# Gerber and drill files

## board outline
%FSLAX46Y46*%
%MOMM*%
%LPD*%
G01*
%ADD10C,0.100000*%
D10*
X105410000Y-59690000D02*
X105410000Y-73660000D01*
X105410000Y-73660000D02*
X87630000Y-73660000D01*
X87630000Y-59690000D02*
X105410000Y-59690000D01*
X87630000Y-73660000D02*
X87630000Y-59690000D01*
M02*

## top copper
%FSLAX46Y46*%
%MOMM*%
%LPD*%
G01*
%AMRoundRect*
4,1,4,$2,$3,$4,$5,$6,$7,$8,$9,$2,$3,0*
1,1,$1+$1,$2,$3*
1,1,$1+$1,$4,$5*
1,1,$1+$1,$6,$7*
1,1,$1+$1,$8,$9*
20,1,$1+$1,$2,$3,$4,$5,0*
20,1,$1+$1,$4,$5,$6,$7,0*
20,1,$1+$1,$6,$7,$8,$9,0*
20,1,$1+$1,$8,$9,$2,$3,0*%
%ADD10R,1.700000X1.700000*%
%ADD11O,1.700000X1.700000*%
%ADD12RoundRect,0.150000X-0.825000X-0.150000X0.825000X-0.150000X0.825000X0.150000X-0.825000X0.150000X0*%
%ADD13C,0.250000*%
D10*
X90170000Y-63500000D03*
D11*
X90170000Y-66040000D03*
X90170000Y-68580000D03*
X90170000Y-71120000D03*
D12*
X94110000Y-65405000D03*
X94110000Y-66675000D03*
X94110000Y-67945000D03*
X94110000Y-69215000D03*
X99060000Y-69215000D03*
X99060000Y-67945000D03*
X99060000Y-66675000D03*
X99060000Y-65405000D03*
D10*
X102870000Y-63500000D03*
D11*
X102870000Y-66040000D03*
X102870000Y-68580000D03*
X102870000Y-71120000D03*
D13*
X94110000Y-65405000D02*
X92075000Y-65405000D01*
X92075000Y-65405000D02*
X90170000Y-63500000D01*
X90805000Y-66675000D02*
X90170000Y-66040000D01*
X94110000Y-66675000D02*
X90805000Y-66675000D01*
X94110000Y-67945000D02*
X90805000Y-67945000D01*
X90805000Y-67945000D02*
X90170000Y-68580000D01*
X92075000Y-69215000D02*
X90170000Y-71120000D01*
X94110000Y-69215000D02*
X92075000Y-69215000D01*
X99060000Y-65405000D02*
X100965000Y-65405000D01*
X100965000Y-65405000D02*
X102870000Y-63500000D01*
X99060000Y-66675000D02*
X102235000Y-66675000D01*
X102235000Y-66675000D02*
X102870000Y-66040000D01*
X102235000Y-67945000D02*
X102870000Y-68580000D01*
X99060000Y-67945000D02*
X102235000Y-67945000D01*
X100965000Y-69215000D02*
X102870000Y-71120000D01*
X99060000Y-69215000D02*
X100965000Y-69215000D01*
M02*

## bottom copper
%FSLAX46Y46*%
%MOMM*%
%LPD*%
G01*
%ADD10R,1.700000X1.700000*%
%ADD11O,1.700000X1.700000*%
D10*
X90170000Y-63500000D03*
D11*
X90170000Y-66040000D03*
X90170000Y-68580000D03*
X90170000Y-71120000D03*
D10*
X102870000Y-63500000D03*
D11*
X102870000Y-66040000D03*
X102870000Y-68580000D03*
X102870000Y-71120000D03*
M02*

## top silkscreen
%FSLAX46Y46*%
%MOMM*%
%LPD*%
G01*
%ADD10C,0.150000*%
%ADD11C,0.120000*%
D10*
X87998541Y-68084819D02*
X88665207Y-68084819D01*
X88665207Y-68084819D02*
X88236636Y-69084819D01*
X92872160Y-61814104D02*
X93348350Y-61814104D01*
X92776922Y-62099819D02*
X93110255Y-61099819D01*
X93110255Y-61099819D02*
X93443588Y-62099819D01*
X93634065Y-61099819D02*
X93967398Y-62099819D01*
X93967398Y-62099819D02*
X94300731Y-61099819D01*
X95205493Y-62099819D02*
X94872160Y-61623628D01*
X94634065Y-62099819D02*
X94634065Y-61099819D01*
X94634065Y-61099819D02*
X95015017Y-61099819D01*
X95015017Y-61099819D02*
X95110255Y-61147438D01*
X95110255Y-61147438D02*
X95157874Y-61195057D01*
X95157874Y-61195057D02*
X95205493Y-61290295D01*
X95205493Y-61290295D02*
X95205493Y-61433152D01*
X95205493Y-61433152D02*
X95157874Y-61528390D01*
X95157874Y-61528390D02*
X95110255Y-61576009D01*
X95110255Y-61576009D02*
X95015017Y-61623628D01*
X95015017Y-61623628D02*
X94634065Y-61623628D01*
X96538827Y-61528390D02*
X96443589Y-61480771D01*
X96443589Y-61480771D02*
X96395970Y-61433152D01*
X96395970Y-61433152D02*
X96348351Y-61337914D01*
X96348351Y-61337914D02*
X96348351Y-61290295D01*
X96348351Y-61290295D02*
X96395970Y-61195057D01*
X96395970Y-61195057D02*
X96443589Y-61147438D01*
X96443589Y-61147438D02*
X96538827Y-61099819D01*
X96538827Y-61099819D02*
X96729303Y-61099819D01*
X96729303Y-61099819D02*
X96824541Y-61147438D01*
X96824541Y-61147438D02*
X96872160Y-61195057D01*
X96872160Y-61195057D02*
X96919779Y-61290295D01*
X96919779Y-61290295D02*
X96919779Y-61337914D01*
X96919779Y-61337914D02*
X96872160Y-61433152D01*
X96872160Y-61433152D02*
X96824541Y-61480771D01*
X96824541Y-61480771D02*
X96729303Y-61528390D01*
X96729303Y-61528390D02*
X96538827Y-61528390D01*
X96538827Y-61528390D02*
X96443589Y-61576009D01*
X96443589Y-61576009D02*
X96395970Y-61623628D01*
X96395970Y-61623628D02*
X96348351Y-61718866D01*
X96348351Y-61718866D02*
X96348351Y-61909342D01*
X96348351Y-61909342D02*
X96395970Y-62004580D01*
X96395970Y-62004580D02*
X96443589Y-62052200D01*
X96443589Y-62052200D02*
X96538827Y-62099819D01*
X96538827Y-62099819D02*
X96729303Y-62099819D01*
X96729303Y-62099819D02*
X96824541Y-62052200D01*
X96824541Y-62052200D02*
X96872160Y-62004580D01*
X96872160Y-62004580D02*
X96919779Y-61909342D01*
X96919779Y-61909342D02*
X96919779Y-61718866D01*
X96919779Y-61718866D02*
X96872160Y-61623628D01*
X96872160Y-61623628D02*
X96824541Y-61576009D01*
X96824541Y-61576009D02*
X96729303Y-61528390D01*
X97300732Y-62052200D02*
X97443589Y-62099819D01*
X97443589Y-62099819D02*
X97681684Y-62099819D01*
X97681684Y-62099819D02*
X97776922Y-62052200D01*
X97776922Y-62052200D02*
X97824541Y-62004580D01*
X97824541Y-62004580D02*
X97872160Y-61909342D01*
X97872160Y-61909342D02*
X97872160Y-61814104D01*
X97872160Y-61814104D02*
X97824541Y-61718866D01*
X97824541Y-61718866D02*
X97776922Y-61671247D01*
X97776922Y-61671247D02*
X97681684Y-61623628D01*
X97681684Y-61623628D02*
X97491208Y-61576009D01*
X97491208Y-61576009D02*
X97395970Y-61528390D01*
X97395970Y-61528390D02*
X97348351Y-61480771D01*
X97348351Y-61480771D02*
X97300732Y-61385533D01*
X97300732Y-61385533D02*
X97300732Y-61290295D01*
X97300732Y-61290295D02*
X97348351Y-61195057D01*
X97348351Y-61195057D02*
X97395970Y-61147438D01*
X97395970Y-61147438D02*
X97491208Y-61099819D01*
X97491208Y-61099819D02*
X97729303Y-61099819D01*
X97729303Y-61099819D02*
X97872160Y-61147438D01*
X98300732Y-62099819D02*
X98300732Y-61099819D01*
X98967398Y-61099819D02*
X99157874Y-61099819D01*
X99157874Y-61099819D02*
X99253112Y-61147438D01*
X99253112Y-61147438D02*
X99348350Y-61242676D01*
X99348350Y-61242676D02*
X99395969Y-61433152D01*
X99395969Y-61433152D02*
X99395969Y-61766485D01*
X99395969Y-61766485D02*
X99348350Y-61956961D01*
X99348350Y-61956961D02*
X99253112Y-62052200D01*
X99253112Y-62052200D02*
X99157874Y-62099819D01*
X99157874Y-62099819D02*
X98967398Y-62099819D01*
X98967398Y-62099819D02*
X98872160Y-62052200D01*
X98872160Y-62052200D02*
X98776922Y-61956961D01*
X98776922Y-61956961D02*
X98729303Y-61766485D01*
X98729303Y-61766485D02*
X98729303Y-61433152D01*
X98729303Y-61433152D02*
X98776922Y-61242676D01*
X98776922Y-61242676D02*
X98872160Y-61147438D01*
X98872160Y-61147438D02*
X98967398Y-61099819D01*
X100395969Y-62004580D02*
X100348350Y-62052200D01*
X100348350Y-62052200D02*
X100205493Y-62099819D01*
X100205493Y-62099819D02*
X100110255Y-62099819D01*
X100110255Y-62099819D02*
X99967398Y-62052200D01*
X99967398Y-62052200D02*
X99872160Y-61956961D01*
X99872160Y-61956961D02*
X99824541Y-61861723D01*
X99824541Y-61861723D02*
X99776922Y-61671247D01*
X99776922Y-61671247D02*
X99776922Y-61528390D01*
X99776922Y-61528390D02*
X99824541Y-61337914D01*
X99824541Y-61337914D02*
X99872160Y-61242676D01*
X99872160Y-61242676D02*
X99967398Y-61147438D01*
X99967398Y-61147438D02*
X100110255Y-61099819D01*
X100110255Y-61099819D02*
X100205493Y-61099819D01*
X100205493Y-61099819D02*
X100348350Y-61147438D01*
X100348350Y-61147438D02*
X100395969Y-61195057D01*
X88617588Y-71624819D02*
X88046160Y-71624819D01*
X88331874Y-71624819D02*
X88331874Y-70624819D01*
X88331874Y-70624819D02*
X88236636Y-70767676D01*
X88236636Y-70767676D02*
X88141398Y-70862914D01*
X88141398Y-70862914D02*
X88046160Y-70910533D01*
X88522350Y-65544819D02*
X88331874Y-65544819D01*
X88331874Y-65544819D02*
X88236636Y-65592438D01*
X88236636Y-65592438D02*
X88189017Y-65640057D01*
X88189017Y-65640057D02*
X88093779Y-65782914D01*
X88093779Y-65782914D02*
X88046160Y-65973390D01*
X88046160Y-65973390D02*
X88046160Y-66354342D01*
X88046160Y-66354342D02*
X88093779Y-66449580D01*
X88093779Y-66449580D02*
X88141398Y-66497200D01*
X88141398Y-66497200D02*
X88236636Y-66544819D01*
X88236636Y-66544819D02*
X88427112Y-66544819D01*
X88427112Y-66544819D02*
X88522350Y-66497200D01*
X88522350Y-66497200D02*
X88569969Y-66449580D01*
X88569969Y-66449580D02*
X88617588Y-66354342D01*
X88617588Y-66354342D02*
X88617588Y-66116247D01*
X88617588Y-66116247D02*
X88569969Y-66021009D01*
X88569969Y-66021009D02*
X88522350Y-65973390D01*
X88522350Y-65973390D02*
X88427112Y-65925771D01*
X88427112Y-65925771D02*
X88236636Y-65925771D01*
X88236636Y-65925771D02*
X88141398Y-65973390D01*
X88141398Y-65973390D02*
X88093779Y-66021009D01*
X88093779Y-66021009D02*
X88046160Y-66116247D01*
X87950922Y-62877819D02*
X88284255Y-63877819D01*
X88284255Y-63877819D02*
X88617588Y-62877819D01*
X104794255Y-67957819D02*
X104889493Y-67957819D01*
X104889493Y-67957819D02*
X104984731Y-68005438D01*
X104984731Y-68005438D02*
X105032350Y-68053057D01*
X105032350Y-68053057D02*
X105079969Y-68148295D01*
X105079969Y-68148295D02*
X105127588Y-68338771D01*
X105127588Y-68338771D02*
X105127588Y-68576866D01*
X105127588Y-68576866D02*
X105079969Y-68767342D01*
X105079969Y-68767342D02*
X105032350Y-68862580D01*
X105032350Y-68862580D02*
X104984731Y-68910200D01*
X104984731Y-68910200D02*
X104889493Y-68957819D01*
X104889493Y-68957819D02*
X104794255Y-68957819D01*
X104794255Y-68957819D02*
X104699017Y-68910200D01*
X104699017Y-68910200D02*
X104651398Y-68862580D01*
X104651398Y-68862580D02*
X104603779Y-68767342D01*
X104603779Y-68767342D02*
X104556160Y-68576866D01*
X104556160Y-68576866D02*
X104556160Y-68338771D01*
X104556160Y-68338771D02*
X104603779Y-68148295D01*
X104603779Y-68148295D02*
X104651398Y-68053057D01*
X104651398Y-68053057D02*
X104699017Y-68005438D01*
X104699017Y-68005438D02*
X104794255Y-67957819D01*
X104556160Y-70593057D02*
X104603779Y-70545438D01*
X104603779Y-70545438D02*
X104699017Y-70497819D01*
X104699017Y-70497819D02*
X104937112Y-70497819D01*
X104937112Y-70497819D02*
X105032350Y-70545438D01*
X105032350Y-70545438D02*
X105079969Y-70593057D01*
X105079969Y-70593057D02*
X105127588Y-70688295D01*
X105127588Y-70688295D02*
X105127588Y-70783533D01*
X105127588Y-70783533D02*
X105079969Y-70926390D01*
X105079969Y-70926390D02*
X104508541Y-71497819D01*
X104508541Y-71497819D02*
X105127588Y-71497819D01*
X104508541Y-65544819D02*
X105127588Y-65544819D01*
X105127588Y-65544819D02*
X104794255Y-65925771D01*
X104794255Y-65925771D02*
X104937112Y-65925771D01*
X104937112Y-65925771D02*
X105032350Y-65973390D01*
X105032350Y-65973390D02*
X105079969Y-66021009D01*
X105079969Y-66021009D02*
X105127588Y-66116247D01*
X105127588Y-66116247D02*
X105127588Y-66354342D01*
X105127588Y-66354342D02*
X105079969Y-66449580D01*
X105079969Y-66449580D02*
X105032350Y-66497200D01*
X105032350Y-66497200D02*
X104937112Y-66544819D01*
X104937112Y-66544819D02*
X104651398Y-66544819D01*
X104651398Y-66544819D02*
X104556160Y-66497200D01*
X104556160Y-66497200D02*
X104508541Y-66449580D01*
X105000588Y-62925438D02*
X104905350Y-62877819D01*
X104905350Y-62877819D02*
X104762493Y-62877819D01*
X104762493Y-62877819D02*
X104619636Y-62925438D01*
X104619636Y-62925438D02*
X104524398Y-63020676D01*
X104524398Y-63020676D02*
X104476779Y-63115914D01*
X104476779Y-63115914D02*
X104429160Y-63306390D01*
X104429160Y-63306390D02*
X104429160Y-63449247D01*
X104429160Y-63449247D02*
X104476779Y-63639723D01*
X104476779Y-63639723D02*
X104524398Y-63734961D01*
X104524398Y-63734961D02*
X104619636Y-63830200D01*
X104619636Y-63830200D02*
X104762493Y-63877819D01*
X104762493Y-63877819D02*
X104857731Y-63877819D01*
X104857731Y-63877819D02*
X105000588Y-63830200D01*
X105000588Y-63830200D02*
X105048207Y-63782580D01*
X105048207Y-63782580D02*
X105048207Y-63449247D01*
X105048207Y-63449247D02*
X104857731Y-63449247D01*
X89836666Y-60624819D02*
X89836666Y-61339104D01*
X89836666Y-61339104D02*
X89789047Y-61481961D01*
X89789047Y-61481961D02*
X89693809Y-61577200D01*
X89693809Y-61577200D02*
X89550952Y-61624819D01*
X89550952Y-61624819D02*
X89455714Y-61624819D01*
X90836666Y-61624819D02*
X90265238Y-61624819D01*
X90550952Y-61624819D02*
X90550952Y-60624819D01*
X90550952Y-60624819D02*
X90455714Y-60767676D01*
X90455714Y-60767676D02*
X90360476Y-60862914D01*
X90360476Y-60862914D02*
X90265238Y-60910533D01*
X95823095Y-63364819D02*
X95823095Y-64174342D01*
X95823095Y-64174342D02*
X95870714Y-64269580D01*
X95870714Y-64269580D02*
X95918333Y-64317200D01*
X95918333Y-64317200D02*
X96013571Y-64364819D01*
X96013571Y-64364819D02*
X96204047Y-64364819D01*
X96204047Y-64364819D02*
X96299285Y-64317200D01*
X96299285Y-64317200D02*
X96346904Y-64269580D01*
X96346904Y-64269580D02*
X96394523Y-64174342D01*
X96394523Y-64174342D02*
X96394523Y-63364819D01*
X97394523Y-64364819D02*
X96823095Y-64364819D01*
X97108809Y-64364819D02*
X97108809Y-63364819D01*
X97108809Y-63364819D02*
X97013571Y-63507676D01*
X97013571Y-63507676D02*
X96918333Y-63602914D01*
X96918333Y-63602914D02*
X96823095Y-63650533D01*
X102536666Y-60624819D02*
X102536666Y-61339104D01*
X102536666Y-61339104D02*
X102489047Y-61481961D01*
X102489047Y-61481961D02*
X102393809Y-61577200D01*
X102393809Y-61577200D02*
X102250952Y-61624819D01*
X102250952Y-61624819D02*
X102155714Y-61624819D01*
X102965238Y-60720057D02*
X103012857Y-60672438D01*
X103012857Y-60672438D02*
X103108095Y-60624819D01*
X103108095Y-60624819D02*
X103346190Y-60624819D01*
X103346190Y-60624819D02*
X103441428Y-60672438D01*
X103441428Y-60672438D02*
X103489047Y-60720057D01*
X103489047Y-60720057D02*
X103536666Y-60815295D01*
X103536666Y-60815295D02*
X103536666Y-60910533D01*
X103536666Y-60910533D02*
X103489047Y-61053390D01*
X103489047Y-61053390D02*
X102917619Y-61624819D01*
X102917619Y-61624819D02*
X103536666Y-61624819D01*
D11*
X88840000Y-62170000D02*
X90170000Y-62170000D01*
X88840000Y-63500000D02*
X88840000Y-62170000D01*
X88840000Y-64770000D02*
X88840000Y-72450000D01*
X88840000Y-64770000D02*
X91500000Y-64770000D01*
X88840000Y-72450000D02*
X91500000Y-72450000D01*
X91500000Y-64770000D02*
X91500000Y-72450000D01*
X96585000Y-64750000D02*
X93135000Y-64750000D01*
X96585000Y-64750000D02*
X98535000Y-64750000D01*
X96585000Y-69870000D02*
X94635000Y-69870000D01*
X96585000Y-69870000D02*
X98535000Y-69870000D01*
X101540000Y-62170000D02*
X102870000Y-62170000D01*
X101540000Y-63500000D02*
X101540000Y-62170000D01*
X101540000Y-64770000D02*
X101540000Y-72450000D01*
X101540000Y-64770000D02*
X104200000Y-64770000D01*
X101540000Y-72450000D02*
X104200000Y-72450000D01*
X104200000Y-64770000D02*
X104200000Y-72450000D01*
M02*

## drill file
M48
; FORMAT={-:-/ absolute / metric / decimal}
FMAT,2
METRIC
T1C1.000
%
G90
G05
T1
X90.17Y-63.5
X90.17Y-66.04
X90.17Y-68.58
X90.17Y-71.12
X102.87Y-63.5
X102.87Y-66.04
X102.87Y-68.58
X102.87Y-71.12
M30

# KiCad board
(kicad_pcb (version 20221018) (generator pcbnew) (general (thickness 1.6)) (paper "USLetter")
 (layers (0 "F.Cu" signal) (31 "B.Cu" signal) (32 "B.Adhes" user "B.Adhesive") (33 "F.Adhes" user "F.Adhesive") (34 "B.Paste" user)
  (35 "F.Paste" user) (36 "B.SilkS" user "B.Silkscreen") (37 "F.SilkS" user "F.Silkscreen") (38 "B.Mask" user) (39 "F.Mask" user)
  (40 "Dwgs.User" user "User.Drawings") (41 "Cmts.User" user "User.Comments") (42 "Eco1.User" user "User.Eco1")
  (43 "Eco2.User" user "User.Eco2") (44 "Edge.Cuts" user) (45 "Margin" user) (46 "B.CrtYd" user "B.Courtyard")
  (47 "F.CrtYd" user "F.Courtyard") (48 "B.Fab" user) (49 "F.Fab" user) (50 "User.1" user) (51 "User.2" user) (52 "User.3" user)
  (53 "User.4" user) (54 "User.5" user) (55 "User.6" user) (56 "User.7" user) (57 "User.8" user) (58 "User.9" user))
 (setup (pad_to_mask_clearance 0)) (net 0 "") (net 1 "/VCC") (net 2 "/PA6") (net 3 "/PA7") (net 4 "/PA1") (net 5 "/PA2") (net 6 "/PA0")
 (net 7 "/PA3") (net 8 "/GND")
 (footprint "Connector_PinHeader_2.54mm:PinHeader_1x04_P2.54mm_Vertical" (layer "F.Cu") (at 90.17 63.5)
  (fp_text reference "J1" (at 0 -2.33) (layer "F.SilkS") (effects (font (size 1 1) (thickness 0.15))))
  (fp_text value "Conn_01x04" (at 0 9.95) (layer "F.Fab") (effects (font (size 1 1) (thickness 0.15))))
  (fp_line (start -1.33 -1.33) (end 0 -1.33) (stroke (width 0.12) (type solid)) (layer "F.SilkS"))
  (fp_line (start -1.33 0) (end -1.33 -1.33) (stroke (width 0.12) (type solid)) (layer "F.SilkS"))
  (fp_line (start -1.33 1.27) (end -1.33 8.95) (stroke (width 0.12) (type solid)) (layer "F.SilkS"))
  (fp_line (start -1.33 1.27) (end 1.33 1.27) (stroke (width 0.12) (type solid)) (layer "F.SilkS"))
  (fp_line (start -1.33 8.95) (end 1.33 8.95) (stroke (width 0.12) (type solid)) (layer "F.SilkS"))
  (fp_line (start 1.33 1.27) (end 1.33 8.95) (stroke (width 0.12) (type solid)) (layer "F.SilkS"))
  (pad "1" thru_hole rect (at 0 0) (size 1.7 1.7) (drill 1) (layers "*.Cu" "*.Mask") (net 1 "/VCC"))
  (pad "2" thru_hole oval (at 0 2.54) (size 1.7 1.7) (drill 1) (layers "*.Cu" "*.Mask") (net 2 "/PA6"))
  (pad "3" thru_hole oval (at 0 5.08) (size 1.7 1.7) (drill 1) (layers "*.Cu" "*.Mask") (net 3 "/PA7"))
  (pad "4" thru_hole oval (at 0 7.62) (size 1.7 1.7) (drill 1) (layers "*.Cu" "*.Mask") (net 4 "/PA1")))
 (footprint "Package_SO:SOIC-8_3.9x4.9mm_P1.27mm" (layer "F.Cu") (at 96.585 67.31)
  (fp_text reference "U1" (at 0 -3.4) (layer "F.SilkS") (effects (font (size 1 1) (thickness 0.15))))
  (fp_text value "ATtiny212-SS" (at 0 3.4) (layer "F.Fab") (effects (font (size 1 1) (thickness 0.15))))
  (fp_line (start 0 -2.56) (end -3.45 -2.56) (stroke (width 0.12) (type solid)) (layer "F.SilkS"))
  (fp_line (start 0 -2.56) (end 1.95 -2.56) (stroke (width 0.12) (type solid)) (layer "F.SilkS"))
  (fp_line (start 0 2.56) (end -1.95 2.56) (stroke (width 0.12) (type solid)) (layer "F.SilkS"))
  (fp_line (start 0 2.56) (end 1.95 2.56) (stroke (width 0.12) (type solid)) (layer "F.SilkS"))
  (pad "1" smd roundrect (at -2.475 -1.905) (size 1.95 0.6) (layers "F.Cu" "F.Paste" "F.Mask") (roundrect_rratio 0.25) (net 1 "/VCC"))
  (pad "2" smd roundrect (at -2.475 -0.635) (size 1.95 0.6) (layers "F.Cu" "F.Paste" "F.Mask") (roundrect_rratio 0.25) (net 2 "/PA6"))
  (pad "3" smd roundrect (at -2.475 0.635) (size 1.95 0.6) (layers "F.Cu" "F.Paste" "F.Mask") (roundrect_rratio 0.25) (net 3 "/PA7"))
  (pad "4" smd roundrect (at -2.475 1.905) (size 1.95 0.6) (layers "F.Cu" "F.Paste" "F.Mask") (roundrect_rratio 0.25) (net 4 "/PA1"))
  (pad "5" smd roundrect (at 2.475 1.905) (size 1.95 0.6) (layers "F.Cu" "F.Paste" "F.Mask") (roundrect_rratio 0.25) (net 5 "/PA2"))
  (pad "6" smd roundrect (at 2.475 0.635) (size 1.95 0.6) (layers "F.Cu" "F.Paste" "F.Mask") (roundrect_rratio 0.25) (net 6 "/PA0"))
  (pad "7" smd roundrect (at 2.475 -0.635) (size 1.95 0.6) (layers "F.Cu" "F.Paste" "F.Mask") (roundrect_rratio 0.25) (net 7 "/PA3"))
  (pad "8" smd roundrect (at 2.475 -1.905) (size 1.95 0.6) (layers "F.Cu" "F.Paste" "F.Mask") (roundrect_rratio 0.25) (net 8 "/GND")))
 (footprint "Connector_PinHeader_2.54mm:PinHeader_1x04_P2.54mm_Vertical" (layer "F.Cu") (at 102.87 63.5)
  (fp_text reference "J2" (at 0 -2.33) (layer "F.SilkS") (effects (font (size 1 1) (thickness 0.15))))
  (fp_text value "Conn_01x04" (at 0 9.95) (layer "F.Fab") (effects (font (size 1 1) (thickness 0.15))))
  (fp_line (start -1.33 -1.33) (end 0 -1.33) (stroke (width 0.12) (type solid)) (layer "F.SilkS"))
  (fp_line (start -1.33 0) (end -1.33 -1.33) (stroke (width 0.12) (type solid)) (layer "F.SilkS"))
  (fp_line (start -1.33 1.27) (end -1.33 8.95) (stroke (width 0.12) (type solid)) (layer "F.SilkS"))
  (fp_line (start -1.33 1.27) (end 1.33 1.27) (stroke (width 0.12) (type solid)) (layer "F.SilkS"))
  (fp_line (start -1.33 8.95) (end 1.33 8.95) (stroke (width 0.12) (type solid)) (layer "F.SilkS"))
  (fp_line (start 1.33 1.27) (end 1.33 8.95) (stroke (width 0.12) (type solid)) (layer "F.SilkS"))
  (pad "1" thru_hole rect (at 0 0) (size 1.7 1.7) (drill 1) (layers "*.Cu" "*.Mask") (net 8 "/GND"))
  (pad "2" thru_hole oval (at 0 2.54) (size 1.7 1.7) (drill 1) (layers "*.Cu" "*.Mask") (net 7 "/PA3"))
  (pad "3" thru_hole oval (at 0 5.08) (size 1.7 1.7) (drill 1) (layers "*.Cu" "*.Mask") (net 6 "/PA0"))
  (pad "4" thru_hole oval (at 0 7.62) (size 1.7 1.7) (drill 1) (layers "*.Cu" "*.Mask") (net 5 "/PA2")))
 (gr_line (start 105.41 59.69) (end 105.41 73.66) (stroke (width 0.1) (type default)) (layer "Edge.Cuts"))
 (gr_line (start 105.41 73.66) (end 87.63 73.66) (stroke (width 0.1) (type default)) (layer "Edge.Cuts"))
 (gr_line (start 87.63 59.69) (end 105.41 59.69) (stroke (width 0.1) (type default)) (layer "Edge.Cuts"))
 (gr_line (start 87.63 73.66) (end 87.63 59.69) (stroke (width 0.1) (type default)) (layer "Edge.Cuts"))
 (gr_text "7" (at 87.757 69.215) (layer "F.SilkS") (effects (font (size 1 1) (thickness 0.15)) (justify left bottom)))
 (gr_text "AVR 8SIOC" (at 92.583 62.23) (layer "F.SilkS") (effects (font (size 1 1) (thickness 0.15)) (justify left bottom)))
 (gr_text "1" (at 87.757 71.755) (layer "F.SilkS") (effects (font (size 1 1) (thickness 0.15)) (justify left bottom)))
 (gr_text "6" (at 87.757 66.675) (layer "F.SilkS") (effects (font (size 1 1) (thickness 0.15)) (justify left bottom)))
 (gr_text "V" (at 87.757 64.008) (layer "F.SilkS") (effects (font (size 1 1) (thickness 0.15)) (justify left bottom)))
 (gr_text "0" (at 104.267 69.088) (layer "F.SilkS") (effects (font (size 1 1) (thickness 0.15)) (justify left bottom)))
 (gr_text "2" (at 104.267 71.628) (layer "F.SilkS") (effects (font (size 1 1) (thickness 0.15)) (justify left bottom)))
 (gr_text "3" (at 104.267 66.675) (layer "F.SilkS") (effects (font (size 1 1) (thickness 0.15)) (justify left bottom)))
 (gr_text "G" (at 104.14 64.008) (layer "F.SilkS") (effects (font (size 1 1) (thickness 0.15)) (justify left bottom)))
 (segment (start 94.11 65.405) (end 92.075 65.405) (width 0.25) (layer "F.Cu") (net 1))
 (segment (start 92.075 65.405) (end 90.17 63.5) (width 0.25) (layer "F.Cu") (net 1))
 (segment (start 90.805 66.675) (end 90.17 66.04) (width 0.25) (layer "F.Cu") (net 2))
 (segment (start 94.11 66.675) (end 90.805 66.675) (width 0.25) (layer "F.Cu") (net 2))
 (segment (start 94.11 67.945) (end 90.805 67.945) (width 0.25) (layer "F.Cu") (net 3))
 (segment (start 90.805 67.945) (end 90.17 68.58) (width 0.25) (layer "F.Cu") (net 3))
 (segment (start 92.075 69.215) (end 90.17 71.12) (width 0.25) (layer "F.Cu") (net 4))
 (segment (start 94.11 69.215) (end 92.075 69.215) (width 0.25) (layer "F.Cu") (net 4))
 (segment (start 99.06 65.405) (end 100.965 65.405) (width 0.25) (layer "F.Cu") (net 8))
 (segment (start 100.965 65.405) (end 102.87 63.5) (width 0.25) (layer "F.Cu") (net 8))
 (segment (start 99.06 66.675) (end 102.235 66.675) (width 0.25) (layer "F.Cu") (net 7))
 (segment (start 102.235 66.675) (end 102.87 66.04) (width 0.25) (layer "F.Cu") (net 7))
 (segment (start 102.235 67.945) (end 102.87 68.58) (width 0.25) (layer "F.Cu") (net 6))
 (segment (start 99.06 67.945) (end 102.235 67.945) (width 0.25) (layer "F.Cu") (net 6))
 (segment (start 100.965 69.215) (end 102.87 71.12) (width 0.25) (layer "F.Cu") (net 5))
 (segment (start 99.06 69.215) (end 100.965 69.215) (width 0.25) (layer "F.Cu") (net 5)))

